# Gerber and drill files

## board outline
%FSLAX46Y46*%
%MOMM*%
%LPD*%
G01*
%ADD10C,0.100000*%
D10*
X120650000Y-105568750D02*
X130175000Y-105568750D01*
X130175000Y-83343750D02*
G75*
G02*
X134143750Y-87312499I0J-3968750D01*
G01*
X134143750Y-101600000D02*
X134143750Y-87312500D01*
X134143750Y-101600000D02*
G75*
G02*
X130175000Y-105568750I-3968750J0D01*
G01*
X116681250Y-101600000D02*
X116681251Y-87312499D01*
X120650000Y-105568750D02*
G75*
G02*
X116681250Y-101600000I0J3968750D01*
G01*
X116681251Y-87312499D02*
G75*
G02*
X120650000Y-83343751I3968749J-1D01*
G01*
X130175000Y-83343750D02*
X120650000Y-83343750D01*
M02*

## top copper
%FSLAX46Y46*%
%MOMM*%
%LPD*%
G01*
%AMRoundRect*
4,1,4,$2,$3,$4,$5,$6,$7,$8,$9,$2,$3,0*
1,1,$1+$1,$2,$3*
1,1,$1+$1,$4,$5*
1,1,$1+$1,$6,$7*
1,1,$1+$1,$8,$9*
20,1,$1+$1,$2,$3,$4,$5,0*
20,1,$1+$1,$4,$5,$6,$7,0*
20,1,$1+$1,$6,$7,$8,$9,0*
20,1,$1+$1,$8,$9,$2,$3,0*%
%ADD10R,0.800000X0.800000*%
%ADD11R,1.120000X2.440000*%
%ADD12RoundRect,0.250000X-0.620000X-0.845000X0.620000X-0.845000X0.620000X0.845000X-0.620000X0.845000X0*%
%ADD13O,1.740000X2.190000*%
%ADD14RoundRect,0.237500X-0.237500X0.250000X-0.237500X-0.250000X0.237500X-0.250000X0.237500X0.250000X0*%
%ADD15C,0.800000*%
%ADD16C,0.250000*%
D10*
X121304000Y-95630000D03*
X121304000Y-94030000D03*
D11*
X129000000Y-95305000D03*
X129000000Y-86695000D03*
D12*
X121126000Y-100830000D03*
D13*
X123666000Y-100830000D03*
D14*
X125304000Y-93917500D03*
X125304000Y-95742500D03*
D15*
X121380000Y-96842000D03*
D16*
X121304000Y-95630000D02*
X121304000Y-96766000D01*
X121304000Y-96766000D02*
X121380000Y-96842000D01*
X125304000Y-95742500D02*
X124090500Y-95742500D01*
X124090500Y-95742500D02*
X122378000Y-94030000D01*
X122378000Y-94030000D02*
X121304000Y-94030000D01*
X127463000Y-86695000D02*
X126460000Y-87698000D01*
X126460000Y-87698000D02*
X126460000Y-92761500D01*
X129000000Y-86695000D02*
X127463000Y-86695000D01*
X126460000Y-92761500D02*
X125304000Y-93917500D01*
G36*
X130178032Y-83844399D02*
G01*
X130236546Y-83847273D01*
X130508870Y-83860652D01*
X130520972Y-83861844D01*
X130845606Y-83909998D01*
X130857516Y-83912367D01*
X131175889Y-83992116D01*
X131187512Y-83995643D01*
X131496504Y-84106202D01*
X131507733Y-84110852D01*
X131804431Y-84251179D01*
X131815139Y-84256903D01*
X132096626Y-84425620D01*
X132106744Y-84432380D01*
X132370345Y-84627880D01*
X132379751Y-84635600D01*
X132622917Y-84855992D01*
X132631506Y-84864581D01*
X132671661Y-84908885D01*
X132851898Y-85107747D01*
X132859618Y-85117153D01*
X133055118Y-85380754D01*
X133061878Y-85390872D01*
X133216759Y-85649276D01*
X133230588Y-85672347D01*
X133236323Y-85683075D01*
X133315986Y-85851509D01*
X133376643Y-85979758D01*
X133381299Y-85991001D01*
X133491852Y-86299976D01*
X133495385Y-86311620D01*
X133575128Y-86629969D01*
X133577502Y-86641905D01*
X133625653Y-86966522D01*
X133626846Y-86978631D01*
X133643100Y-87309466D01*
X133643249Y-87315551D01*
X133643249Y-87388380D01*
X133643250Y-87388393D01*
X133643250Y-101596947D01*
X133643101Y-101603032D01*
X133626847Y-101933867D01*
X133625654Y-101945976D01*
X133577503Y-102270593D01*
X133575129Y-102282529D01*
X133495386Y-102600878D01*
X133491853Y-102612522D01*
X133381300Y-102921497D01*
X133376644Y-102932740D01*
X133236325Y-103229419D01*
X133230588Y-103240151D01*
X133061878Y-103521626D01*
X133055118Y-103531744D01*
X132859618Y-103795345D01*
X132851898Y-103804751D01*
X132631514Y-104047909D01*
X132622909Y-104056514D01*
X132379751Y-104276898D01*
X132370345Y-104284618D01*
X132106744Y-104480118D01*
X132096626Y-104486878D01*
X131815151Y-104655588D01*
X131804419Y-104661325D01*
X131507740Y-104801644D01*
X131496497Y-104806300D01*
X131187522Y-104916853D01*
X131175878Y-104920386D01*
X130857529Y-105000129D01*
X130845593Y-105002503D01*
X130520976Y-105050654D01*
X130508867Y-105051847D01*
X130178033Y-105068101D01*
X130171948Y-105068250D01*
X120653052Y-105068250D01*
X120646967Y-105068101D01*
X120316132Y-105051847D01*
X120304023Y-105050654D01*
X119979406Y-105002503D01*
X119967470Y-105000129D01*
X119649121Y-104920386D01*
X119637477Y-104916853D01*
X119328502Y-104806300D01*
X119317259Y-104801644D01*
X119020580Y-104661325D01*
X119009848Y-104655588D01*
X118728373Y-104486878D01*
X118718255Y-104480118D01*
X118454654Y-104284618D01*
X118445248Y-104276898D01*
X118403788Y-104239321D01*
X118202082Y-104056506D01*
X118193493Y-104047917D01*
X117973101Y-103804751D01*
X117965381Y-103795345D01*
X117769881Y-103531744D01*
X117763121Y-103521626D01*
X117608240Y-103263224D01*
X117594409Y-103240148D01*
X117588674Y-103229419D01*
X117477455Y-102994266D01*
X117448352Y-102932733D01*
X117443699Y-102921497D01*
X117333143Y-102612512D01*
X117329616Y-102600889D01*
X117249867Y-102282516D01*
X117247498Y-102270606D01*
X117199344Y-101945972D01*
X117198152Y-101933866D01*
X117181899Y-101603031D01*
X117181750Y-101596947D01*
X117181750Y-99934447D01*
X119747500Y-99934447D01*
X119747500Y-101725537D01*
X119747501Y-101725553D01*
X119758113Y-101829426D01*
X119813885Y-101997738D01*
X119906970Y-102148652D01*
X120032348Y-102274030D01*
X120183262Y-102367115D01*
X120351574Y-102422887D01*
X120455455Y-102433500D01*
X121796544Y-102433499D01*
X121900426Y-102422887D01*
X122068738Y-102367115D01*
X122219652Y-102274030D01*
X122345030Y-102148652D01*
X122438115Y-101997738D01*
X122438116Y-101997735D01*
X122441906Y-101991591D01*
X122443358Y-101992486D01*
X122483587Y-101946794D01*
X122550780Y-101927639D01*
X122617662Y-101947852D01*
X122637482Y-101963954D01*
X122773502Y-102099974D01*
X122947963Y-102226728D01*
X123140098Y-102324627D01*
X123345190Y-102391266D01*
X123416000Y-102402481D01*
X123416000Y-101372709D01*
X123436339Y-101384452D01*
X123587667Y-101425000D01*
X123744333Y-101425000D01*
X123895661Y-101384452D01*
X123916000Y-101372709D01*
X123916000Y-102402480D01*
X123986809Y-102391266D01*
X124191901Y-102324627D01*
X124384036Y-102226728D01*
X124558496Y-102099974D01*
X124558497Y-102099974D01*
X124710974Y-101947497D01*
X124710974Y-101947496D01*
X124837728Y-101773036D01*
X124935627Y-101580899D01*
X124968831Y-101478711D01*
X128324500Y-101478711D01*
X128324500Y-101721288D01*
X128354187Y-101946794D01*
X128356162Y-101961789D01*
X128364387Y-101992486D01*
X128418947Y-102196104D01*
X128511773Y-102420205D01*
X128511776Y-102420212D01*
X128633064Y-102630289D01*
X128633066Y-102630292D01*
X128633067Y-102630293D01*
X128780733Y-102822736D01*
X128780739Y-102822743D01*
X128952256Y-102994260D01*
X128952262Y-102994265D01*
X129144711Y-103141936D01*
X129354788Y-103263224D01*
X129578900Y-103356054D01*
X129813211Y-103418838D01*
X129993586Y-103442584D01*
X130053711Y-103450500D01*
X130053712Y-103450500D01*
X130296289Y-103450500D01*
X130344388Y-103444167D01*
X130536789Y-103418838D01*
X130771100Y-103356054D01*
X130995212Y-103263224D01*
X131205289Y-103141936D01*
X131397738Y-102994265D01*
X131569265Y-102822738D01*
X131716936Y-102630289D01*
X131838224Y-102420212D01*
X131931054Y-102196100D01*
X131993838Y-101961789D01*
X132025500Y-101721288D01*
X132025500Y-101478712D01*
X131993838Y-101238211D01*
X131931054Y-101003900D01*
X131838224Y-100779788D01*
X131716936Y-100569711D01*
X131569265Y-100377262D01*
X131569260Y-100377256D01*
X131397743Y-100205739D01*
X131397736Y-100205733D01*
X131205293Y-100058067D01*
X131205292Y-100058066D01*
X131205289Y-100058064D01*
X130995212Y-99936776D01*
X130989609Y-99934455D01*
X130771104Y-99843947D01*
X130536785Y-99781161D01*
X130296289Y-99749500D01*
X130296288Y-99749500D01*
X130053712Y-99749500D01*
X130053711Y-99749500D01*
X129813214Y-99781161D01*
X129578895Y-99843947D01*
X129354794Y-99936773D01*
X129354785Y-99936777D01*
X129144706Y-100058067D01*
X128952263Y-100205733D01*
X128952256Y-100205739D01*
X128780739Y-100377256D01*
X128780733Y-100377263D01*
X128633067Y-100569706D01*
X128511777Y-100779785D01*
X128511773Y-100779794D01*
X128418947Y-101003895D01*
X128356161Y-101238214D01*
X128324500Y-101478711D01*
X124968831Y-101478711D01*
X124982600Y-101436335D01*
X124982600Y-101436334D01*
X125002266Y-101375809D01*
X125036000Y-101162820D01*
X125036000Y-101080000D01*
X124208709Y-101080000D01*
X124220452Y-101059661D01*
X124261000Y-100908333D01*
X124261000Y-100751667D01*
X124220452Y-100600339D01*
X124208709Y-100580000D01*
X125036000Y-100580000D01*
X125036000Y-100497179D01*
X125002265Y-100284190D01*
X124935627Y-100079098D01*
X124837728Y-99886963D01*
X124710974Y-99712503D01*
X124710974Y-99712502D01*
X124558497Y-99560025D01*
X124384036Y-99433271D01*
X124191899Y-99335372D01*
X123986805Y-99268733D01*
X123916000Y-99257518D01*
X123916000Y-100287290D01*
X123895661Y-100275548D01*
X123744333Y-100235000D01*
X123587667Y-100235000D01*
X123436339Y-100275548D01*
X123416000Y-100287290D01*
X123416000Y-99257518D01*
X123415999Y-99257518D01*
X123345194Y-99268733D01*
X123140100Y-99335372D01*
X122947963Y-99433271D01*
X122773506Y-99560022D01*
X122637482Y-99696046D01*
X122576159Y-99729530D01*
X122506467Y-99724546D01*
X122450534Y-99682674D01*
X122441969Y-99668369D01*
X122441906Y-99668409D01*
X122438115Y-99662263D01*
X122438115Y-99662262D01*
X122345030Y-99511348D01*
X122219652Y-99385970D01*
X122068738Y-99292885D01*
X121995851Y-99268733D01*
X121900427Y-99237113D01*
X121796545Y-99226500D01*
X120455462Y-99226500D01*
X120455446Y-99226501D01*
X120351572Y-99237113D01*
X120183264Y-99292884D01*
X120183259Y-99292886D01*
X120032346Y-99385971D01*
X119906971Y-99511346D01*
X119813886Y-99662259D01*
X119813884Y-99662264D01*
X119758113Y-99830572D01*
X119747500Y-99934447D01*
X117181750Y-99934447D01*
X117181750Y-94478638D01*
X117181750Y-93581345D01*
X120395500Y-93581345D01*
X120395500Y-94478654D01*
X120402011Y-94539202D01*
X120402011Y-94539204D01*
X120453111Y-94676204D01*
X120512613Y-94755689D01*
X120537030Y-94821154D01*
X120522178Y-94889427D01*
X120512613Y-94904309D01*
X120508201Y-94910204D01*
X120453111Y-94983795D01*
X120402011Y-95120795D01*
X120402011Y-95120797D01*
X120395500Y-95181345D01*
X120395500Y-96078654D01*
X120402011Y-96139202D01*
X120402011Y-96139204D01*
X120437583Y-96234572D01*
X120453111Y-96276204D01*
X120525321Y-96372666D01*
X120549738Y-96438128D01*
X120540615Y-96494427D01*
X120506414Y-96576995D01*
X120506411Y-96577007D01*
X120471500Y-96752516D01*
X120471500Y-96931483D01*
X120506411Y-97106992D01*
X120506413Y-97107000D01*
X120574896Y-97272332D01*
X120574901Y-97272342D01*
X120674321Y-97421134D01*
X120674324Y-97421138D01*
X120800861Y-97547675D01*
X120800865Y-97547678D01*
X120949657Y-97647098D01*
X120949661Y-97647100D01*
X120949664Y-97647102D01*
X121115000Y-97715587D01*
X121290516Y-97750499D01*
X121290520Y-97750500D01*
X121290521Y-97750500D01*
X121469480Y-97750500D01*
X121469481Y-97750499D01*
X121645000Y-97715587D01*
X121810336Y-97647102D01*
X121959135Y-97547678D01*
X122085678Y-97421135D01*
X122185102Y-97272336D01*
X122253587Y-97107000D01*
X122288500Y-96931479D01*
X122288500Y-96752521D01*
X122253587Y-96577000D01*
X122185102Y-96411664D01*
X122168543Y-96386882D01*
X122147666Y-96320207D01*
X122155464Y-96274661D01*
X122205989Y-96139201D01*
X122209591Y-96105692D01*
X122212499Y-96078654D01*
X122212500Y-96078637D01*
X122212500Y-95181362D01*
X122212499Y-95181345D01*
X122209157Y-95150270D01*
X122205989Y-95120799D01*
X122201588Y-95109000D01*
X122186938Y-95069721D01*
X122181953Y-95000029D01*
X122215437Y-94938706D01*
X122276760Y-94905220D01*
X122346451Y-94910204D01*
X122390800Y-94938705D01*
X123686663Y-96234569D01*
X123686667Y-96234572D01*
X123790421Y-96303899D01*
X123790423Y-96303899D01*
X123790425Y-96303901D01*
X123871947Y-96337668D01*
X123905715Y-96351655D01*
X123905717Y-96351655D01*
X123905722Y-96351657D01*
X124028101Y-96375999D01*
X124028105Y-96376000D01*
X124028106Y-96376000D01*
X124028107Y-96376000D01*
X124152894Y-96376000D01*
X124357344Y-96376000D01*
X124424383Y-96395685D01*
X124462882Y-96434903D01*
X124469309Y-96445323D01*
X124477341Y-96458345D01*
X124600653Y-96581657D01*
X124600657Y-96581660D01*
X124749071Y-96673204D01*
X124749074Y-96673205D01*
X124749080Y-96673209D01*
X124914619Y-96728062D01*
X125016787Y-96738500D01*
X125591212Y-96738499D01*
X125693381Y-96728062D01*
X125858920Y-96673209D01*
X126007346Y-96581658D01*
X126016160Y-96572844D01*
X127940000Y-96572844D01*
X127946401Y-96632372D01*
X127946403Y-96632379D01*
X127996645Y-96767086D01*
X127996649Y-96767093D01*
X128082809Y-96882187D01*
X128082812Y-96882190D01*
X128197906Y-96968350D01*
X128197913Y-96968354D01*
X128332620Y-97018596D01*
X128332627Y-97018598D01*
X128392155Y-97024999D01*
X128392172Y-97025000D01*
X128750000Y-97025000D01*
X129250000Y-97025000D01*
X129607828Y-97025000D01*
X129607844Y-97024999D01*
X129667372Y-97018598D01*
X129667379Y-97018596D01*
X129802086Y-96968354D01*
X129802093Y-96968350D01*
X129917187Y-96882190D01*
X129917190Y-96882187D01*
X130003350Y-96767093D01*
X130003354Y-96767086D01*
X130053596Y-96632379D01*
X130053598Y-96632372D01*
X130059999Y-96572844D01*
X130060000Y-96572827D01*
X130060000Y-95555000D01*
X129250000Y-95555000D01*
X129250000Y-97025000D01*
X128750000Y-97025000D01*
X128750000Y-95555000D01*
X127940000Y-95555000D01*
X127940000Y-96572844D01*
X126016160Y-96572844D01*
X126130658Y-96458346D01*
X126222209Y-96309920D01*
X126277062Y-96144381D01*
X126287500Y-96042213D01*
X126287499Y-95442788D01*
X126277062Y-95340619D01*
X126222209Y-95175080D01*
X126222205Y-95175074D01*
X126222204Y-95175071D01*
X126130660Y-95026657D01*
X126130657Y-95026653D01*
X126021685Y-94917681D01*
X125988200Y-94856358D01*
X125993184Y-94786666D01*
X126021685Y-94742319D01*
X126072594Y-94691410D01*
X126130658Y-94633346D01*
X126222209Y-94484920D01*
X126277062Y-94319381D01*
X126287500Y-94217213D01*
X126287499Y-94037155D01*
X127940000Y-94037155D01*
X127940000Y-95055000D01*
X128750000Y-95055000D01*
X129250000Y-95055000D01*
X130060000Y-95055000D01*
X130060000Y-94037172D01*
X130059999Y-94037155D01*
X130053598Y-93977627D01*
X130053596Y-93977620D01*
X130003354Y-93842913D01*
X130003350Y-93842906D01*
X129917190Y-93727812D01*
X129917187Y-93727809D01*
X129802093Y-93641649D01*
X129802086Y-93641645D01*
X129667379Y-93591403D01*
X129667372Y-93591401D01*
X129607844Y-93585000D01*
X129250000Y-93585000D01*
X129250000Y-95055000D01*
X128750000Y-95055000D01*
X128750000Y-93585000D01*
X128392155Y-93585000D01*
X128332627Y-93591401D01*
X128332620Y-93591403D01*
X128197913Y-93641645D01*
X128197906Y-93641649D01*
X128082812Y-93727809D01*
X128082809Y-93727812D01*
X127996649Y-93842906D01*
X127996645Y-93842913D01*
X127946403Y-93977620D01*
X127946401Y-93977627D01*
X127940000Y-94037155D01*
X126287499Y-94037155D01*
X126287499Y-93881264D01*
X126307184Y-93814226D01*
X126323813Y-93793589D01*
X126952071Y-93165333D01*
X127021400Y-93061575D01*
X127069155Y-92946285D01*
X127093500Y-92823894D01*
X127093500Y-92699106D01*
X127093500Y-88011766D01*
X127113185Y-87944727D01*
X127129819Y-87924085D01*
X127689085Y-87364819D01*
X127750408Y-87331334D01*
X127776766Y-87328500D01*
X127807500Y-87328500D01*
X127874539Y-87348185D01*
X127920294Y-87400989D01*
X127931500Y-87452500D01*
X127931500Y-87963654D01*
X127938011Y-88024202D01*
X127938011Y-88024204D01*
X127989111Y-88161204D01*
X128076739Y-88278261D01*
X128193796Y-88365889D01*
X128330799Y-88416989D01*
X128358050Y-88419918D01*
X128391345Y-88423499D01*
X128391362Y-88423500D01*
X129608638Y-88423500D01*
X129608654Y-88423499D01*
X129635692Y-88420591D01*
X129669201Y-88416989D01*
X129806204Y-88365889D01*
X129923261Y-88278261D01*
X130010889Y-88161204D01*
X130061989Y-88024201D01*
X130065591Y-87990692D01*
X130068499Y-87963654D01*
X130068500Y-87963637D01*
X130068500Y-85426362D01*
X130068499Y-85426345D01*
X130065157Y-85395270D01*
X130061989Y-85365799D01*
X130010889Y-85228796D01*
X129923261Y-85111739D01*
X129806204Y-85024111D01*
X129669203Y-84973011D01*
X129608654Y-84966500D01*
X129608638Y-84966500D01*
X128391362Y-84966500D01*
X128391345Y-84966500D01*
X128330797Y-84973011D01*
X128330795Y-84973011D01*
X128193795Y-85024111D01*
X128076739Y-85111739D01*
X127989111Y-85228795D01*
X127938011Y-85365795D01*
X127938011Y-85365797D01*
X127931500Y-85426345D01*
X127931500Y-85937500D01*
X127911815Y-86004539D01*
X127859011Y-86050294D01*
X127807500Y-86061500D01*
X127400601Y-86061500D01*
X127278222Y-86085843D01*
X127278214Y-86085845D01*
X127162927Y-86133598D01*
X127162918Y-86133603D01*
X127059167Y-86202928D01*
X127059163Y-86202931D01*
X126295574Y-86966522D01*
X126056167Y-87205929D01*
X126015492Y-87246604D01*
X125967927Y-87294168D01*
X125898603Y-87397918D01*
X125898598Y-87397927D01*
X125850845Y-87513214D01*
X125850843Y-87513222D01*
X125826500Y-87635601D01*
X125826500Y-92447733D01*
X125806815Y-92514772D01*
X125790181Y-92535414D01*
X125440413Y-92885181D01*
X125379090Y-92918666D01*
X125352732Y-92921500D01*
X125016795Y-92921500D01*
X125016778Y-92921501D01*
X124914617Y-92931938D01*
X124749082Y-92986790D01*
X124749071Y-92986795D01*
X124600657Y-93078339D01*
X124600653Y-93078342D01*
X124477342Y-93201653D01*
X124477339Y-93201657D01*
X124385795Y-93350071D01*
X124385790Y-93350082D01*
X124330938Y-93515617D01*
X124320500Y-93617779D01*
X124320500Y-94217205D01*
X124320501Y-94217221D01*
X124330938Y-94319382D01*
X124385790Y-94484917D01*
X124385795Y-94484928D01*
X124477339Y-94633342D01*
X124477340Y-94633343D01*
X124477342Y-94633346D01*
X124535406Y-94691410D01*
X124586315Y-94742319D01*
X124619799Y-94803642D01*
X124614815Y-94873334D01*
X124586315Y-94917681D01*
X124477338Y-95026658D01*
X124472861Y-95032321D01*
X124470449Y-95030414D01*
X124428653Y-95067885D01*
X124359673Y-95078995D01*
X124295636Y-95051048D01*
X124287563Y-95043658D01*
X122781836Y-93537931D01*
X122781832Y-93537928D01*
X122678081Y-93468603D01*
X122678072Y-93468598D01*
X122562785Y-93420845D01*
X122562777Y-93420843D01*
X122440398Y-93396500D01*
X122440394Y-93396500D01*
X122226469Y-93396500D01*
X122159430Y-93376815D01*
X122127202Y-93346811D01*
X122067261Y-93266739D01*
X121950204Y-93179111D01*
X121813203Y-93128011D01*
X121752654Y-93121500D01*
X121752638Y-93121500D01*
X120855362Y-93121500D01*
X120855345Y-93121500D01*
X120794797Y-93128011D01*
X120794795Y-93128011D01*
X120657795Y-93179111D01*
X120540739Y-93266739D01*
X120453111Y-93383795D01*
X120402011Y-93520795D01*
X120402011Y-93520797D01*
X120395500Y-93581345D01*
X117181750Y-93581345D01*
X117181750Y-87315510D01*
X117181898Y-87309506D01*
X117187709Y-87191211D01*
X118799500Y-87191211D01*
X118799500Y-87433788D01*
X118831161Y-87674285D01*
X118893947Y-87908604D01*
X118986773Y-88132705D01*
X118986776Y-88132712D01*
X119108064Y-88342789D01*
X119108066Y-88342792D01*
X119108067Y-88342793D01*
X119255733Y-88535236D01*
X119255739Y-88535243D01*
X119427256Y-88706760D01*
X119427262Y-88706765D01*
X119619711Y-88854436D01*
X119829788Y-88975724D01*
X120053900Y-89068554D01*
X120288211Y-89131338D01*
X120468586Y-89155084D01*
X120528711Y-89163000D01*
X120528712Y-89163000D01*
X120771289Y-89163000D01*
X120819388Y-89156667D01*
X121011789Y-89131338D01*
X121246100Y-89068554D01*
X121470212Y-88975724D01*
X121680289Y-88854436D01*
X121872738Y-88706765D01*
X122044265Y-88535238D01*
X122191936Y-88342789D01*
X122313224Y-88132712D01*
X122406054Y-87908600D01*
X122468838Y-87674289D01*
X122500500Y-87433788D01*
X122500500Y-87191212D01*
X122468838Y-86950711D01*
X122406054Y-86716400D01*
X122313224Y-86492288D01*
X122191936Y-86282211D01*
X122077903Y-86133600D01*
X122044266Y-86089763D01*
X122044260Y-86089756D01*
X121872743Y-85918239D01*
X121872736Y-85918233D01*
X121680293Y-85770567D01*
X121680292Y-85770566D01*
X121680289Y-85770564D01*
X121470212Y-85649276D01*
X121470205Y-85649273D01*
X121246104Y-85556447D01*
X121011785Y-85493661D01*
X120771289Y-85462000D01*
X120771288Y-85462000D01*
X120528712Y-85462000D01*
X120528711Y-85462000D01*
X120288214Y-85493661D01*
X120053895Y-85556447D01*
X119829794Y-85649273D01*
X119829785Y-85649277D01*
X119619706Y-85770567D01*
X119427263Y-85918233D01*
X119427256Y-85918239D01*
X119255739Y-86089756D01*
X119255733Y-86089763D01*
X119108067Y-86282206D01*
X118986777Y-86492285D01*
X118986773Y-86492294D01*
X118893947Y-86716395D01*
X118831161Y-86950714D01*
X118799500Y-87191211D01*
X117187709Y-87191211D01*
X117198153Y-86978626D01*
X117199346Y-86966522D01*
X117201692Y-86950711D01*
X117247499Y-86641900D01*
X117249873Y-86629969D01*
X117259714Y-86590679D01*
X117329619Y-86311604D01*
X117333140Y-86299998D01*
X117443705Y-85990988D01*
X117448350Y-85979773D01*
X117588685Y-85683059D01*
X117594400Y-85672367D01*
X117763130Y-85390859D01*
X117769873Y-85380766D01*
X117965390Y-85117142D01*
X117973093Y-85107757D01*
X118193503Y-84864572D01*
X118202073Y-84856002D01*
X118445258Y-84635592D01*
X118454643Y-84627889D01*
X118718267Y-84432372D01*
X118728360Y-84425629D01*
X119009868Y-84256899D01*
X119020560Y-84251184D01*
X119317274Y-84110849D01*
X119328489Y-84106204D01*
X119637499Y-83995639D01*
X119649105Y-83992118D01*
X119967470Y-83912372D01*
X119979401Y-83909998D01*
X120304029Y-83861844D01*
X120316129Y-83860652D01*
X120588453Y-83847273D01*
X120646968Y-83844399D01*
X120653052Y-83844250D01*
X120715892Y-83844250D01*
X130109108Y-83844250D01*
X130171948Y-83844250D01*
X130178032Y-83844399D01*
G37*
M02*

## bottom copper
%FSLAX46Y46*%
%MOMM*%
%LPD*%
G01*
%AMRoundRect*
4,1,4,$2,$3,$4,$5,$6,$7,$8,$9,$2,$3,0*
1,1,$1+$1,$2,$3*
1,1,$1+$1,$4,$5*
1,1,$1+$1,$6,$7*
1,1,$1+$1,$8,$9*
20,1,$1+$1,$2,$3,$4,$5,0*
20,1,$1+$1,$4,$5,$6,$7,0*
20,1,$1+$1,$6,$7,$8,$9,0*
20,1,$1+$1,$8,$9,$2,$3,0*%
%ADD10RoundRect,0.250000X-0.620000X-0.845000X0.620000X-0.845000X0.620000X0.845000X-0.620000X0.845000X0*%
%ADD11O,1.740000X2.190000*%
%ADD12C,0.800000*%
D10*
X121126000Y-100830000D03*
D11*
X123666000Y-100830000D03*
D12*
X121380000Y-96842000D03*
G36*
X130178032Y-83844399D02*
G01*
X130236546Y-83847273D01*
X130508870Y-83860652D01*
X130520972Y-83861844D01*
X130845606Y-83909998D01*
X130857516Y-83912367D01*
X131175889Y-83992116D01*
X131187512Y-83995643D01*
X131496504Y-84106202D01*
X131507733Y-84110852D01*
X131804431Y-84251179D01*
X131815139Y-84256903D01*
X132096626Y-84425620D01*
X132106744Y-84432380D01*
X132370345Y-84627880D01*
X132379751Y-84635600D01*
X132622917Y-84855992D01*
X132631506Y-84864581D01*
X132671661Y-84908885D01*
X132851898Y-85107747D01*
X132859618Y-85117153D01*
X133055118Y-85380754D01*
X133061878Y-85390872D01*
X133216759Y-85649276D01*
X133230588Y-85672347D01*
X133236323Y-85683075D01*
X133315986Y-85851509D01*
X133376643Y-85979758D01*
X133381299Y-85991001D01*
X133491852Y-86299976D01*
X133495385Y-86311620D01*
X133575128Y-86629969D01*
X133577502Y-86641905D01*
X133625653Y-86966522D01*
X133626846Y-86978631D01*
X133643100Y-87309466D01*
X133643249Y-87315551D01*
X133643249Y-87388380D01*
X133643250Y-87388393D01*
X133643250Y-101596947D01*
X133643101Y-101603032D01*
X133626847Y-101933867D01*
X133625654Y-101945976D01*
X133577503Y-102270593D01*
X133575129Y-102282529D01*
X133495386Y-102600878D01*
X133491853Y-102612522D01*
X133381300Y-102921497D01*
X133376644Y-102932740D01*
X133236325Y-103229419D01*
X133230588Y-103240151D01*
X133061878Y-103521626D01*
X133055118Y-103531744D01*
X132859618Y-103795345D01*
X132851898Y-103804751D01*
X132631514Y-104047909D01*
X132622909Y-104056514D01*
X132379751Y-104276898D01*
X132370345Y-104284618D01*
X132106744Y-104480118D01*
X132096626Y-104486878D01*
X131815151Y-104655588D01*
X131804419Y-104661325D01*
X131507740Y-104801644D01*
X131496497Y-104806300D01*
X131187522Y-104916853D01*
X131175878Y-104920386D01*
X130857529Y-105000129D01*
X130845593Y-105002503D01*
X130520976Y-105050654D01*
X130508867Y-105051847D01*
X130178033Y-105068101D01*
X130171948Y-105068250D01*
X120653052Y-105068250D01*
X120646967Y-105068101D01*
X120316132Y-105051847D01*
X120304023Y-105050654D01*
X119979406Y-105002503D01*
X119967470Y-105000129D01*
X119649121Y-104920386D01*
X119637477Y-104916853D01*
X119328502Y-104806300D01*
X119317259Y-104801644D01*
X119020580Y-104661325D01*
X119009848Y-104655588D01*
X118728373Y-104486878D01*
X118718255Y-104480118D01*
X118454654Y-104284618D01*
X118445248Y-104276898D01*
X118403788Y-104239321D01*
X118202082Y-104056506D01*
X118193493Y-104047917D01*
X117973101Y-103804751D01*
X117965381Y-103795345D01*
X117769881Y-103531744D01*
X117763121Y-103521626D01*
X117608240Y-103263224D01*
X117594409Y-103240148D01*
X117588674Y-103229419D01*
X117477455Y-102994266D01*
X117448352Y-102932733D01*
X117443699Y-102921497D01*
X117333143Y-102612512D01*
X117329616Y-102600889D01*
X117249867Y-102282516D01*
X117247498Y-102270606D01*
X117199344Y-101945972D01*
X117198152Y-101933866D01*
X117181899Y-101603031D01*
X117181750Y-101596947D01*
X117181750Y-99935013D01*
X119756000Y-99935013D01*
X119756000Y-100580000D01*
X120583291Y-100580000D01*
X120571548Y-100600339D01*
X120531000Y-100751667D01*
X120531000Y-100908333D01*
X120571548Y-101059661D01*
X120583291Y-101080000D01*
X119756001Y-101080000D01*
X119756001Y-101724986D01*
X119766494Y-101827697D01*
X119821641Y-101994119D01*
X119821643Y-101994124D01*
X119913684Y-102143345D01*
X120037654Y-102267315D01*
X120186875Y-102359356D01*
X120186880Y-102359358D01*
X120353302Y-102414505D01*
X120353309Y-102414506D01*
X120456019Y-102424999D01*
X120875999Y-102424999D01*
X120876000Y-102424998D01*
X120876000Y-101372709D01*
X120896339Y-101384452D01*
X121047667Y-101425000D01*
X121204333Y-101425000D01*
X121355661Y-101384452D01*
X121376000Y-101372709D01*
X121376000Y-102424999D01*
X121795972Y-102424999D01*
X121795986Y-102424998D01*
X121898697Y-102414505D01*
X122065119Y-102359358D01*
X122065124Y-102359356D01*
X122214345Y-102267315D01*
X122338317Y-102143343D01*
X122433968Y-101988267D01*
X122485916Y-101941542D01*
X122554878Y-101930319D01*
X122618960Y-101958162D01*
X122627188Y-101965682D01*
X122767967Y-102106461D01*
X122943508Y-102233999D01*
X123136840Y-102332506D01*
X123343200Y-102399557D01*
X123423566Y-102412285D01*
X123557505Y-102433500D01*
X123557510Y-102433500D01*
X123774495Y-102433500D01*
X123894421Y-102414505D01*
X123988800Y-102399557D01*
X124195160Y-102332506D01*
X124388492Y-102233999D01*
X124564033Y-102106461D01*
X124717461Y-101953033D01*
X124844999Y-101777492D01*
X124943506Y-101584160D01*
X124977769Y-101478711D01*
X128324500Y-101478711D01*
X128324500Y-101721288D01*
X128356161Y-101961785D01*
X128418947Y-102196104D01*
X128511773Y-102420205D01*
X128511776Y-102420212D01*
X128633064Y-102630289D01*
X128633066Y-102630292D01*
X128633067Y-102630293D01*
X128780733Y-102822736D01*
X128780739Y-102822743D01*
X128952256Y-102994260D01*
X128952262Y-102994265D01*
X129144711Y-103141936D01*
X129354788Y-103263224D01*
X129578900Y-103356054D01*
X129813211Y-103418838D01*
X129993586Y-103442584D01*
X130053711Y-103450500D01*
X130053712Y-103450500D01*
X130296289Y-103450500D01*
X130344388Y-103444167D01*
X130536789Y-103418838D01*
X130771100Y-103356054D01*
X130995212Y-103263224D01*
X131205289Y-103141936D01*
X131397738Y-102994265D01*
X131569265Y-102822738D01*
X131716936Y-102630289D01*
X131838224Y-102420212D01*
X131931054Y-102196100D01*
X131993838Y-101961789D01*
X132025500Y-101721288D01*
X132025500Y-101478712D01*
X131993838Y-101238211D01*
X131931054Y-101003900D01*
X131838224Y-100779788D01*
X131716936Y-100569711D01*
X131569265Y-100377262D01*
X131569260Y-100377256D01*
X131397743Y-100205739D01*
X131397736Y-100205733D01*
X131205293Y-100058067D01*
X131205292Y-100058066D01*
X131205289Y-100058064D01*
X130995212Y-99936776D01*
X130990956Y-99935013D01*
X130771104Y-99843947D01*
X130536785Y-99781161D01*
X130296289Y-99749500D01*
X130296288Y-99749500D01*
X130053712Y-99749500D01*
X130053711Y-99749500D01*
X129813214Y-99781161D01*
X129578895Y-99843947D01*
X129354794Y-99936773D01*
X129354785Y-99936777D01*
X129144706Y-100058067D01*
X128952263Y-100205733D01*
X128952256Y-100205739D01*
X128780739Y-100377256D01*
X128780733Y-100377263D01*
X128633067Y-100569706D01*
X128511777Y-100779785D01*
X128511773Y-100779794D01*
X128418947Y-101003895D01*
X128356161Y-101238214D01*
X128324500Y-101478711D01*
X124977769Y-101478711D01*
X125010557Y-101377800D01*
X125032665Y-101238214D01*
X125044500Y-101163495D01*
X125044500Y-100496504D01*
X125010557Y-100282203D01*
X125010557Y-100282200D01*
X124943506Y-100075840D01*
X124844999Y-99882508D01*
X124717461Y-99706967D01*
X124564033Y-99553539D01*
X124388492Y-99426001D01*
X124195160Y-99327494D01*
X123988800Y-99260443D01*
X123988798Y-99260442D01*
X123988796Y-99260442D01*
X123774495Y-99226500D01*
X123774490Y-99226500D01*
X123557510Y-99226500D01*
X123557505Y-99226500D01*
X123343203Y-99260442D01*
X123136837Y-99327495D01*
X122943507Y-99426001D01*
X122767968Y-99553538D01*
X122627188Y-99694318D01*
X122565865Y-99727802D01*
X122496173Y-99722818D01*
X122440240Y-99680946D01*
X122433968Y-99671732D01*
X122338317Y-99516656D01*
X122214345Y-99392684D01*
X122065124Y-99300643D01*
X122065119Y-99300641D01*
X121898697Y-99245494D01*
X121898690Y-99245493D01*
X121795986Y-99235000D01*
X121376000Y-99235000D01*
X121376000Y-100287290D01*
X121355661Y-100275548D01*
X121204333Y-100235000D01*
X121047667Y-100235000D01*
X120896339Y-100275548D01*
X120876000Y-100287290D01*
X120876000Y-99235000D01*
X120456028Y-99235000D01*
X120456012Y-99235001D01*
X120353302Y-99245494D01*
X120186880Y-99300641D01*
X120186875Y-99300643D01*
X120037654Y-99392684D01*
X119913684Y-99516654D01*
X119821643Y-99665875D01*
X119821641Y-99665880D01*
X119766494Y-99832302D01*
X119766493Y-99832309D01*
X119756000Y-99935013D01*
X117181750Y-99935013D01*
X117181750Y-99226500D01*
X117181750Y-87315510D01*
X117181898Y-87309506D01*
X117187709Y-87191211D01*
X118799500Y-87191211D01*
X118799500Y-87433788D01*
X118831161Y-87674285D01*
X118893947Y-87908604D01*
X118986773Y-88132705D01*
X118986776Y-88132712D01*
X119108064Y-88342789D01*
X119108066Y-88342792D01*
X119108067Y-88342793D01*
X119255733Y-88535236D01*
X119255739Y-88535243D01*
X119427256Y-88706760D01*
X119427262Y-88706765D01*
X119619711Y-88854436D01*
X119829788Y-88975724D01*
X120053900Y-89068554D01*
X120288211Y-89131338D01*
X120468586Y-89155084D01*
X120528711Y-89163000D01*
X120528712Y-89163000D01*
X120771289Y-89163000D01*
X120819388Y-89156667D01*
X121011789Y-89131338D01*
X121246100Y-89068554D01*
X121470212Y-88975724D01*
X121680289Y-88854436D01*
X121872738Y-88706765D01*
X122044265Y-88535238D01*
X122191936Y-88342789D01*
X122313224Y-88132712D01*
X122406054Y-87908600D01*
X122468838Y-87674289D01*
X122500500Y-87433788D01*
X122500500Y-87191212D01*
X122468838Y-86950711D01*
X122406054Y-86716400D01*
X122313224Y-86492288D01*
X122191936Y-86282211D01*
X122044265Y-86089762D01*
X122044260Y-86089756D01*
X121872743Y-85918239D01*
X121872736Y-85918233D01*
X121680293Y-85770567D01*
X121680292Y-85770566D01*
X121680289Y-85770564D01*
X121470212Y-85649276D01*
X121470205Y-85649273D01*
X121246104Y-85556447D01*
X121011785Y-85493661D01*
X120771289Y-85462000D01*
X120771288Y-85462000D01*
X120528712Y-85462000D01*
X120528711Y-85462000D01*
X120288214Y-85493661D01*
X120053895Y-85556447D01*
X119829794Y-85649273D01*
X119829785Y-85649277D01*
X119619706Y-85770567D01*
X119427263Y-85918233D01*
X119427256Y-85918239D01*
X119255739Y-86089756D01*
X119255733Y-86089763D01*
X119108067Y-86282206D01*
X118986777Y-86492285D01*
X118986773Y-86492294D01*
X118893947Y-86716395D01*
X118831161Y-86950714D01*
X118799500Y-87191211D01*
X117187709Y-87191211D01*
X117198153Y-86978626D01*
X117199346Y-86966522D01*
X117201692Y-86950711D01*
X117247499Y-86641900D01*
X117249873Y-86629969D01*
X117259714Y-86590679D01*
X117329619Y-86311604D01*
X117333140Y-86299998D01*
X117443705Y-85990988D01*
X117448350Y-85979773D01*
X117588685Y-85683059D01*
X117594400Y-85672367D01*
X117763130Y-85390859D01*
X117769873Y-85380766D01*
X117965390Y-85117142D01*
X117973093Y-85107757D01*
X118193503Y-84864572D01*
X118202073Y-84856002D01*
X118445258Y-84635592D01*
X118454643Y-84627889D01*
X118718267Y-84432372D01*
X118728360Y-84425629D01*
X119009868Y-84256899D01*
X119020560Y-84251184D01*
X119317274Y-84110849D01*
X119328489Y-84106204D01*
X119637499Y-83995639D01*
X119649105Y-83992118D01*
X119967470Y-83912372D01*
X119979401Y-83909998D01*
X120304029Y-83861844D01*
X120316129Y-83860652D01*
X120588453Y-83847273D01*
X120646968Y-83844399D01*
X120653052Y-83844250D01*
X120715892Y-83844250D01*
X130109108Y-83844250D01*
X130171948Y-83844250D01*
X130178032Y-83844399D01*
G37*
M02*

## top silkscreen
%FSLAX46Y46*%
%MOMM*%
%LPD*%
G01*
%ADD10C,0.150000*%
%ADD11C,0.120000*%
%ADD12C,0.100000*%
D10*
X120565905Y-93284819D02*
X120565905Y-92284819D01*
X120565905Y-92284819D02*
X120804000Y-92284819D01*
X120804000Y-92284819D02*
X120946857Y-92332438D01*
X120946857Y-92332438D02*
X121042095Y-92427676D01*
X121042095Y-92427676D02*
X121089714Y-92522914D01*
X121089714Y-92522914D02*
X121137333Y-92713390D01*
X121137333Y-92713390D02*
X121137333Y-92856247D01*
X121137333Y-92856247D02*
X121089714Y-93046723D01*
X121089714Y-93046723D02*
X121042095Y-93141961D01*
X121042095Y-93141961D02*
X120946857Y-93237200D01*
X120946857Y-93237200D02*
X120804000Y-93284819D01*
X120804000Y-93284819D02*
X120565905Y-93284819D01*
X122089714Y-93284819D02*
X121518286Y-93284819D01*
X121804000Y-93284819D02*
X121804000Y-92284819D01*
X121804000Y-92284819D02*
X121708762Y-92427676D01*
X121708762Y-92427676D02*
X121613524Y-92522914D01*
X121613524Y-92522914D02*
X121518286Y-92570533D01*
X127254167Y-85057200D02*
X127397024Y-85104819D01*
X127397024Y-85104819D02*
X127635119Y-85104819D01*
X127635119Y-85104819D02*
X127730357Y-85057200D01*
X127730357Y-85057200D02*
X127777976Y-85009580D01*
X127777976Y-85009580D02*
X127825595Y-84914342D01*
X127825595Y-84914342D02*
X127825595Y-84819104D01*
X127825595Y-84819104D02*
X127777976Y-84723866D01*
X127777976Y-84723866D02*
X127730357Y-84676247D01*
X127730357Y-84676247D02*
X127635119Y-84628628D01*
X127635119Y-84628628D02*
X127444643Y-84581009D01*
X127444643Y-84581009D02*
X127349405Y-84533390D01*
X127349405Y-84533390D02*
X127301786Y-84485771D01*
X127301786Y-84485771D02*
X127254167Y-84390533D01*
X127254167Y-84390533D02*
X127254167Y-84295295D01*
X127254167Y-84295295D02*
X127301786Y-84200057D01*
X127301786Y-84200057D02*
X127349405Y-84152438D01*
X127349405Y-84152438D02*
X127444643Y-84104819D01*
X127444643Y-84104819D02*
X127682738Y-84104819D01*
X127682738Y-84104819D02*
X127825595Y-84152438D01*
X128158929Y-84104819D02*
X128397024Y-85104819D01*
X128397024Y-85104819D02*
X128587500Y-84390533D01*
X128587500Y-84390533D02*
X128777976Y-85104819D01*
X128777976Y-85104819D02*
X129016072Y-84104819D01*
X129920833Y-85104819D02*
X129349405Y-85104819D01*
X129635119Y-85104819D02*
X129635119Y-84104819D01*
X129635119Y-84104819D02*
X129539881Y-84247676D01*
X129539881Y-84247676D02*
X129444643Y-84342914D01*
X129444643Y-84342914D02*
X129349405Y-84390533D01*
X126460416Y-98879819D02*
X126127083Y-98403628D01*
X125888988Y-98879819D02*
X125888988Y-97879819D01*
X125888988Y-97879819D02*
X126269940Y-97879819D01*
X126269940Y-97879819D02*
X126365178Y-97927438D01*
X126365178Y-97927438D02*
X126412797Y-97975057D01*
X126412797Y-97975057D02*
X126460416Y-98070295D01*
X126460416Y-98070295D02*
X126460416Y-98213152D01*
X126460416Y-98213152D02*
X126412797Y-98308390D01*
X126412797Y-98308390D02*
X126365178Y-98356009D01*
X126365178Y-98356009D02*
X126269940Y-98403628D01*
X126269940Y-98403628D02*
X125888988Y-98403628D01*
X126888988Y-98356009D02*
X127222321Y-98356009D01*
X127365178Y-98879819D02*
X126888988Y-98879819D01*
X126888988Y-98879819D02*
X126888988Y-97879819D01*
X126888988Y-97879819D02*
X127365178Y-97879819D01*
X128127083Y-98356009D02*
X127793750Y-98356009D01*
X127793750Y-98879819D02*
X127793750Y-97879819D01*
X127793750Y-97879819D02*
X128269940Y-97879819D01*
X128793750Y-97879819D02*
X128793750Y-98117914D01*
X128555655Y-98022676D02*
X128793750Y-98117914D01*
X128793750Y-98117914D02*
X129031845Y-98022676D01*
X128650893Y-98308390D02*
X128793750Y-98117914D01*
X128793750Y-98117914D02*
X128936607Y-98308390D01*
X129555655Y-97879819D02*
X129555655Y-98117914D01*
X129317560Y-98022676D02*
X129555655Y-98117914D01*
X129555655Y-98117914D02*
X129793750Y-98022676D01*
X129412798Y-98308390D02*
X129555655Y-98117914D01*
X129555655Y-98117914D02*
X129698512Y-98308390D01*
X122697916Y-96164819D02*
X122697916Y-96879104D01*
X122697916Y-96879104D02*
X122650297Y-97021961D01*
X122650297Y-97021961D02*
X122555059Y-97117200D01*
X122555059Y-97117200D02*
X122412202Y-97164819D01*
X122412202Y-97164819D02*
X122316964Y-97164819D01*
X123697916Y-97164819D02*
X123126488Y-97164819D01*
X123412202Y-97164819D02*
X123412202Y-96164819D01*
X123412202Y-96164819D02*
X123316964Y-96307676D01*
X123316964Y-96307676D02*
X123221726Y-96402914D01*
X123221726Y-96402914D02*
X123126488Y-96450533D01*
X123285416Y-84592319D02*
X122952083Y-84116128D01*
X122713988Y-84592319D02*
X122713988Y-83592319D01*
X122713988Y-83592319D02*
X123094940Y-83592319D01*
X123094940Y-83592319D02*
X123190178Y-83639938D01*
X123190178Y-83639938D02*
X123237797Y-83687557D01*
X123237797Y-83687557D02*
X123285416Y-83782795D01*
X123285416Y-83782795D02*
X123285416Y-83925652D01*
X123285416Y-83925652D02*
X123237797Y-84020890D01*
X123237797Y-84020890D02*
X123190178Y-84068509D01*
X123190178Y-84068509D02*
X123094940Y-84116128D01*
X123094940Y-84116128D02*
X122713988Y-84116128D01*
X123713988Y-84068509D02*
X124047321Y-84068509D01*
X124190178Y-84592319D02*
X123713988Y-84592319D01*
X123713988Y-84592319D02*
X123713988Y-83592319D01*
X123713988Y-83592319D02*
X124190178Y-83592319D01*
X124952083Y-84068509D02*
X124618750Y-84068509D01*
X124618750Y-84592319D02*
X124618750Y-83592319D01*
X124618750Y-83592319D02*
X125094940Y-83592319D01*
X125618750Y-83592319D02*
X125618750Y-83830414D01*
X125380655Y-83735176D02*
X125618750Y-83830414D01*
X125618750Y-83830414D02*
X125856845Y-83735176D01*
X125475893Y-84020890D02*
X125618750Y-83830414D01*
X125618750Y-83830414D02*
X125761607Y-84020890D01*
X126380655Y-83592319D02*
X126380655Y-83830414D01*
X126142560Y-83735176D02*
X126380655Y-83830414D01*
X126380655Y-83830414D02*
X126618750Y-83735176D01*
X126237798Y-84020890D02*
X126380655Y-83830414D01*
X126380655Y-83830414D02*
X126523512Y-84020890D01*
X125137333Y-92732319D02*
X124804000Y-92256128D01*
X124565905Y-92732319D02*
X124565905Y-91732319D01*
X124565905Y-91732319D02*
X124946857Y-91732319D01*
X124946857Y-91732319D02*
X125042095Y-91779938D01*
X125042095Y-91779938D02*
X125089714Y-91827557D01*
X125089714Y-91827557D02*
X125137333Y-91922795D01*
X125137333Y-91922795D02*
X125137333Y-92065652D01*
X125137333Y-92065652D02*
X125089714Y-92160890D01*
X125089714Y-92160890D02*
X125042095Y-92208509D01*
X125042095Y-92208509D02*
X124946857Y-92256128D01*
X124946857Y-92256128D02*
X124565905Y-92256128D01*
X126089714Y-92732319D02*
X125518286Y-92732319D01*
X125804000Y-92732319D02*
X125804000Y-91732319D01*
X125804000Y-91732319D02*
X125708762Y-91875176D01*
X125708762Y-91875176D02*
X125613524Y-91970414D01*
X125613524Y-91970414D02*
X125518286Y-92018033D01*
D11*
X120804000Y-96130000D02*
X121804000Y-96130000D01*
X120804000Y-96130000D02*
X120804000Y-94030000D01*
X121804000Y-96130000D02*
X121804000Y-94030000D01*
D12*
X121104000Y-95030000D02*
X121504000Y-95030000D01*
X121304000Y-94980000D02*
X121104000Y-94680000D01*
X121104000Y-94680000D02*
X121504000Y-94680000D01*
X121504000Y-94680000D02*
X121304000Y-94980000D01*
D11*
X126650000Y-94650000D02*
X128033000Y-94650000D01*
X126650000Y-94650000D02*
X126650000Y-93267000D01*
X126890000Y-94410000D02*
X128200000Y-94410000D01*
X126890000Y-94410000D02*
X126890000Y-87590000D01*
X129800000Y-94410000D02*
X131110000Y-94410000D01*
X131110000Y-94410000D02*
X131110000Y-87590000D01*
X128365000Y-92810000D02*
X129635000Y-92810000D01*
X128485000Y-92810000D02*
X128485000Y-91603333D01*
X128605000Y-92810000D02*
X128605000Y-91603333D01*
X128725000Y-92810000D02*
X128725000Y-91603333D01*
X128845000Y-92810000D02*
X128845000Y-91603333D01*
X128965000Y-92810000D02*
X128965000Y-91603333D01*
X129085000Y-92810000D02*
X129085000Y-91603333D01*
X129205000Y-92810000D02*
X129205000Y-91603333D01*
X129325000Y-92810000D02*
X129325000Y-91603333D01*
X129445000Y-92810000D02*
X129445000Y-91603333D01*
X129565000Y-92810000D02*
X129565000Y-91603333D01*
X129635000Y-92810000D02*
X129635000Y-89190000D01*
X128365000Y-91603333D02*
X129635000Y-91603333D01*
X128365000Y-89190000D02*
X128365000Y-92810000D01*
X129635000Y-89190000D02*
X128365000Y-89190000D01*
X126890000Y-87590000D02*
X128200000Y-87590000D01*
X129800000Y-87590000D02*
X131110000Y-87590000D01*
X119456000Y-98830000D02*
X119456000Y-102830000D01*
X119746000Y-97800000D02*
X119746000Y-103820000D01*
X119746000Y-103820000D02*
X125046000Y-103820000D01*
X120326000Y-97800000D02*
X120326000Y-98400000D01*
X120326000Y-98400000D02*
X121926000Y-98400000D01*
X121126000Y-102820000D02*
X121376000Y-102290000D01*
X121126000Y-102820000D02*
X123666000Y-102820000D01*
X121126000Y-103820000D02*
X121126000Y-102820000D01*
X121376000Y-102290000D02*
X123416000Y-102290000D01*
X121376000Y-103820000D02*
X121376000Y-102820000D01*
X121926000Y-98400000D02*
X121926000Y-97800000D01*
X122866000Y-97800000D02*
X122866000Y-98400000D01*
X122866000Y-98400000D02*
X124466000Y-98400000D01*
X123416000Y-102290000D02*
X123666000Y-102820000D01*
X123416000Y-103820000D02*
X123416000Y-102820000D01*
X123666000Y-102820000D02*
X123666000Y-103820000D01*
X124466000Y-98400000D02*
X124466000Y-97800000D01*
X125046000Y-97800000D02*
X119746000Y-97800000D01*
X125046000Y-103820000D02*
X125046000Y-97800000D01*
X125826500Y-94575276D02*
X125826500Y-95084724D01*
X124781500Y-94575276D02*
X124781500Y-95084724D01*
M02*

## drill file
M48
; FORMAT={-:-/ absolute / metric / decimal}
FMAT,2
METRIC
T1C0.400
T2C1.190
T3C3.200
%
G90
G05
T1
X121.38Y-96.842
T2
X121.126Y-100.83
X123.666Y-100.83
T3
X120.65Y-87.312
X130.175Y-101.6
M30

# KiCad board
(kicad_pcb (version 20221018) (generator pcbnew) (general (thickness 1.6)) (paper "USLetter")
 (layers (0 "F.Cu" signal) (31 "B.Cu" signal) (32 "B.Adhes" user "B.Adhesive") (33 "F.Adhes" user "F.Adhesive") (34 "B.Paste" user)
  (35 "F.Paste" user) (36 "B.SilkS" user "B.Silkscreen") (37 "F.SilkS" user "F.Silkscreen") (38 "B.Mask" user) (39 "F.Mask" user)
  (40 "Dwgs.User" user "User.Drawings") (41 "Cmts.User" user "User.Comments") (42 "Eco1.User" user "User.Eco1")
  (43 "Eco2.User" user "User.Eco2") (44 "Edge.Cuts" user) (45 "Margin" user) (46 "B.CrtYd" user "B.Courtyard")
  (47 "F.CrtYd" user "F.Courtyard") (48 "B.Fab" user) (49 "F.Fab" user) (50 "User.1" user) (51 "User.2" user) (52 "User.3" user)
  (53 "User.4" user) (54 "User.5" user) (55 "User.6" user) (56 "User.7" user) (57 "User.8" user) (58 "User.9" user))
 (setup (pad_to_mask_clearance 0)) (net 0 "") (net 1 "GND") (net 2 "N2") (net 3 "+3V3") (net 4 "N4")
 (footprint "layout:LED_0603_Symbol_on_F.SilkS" (layer "F.Cu") (at 121.304 94.83 90)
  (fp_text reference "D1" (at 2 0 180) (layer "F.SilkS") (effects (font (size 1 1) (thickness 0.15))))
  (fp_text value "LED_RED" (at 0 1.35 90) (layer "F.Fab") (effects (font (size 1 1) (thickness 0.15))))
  (fp_line (start -1.3 -0.5) (end -1.3 0.5) (stroke (width 0.12) (type solid)) (layer "F.SilkS"))
  (fp_line (start -1.3 -0.5) (end 0.8 -0.5) (stroke (width 0.12) (type solid)) (layer "F.SilkS"))
  (fp_line (start -1.3 0.5) (end 0.8 0.5) (stroke (width 0.12) (type solid)) (layer "F.SilkS"))
  (fp_line (start -0.2 -0.2) (end -0.2 0.2) (stroke (width 0.1) (type solid)) (layer "F.SilkS"))
  (fp_line (start -0.15 0) (end 0.15 -0.2) (stroke (width 0.1) (type solid)) (layer "F.SilkS"))
  (fp_line (start 0.15 -0.2) (end 0.15 0.2) (stroke (width 0.1) (type solid)) (layer "F.SilkS"))
  (fp_line (start 0.15 0.2) (end -0.15 0) (stroke (width 0.1) (type solid)) (layer "F.SilkS"))
  (pad "1" smd rect (at -0.8 0 270) (size 0.8 0.8) (layers "F.Cu" "F.Paste" "F.Mask") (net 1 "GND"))
  (pad "2" smd rect (at 0.8 0 270) (size 0.8 0.8) (layers "F.Cu" "F.Paste" "F.Mask") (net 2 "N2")))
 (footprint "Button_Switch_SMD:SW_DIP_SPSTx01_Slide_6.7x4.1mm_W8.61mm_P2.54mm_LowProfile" (layer "F.Cu") (at 129 91 90)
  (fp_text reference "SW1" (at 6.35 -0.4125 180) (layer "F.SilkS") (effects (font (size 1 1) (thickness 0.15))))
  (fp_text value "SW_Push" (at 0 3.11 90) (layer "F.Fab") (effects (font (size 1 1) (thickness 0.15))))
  (fp_line (start -3.65 -2.35) (end -3.65 -0.967) (stroke (width 0.12) (type solid)) (layer "F.SilkS"))
  (fp_line (start -3.65 -2.35) (end -2.267 -2.35) (stroke (width 0.12) (type solid)) (layer "F.SilkS"))
  (fp_line (start -3.41 -2.11) (end -3.41 -0.8) (stroke (width 0.12) (type solid)) (layer "F.SilkS"))
  (fp_line (start -3.41 -2.11) (end 3.41 -2.11) (stroke (width 0.12) (type solid)) (layer "F.SilkS"))
  (fp_line (start -3.41 0.8) (end -3.41 2.11) (stroke (width 0.12) (type solid)) (layer "F.SilkS"))
  (fp_line (start -3.41 2.11) (end 3.41 2.11) (stroke (width 0.12) (type solid)) (layer "F.SilkS"))
  (fp_line (start -1.81 -0.635) (end -1.81 0.635) (stroke (width 0.12) (type solid)) (layer "F.SilkS"))
  (fp_line (start -1.81 -0.515) (end -0.603333 -0.515) (stroke (width 0.12) (type solid)) (layer "F.SilkS"))
  (fp_line (start -1.81 -0.395) (end -0.603333 -0.395) (stroke (width 0.12) (type solid)) (layer "F.SilkS"))
  (fp_line (start -1.81 -0.275) (end -0.603333 -0.275) (stroke (width 0.12) (type solid)) (layer "F.SilkS"))
  (fp_line (start -1.81 -0.155) (end -0.603333 -0.155) (stroke (width 0.12) (type solid)) (layer "F.SilkS"))
  (fp_line (start -1.81 -0.035) (end -0.603333 -0.035) (stroke (width 0.12) (type solid)) (layer "F.SilkS"))
  (fp_line (start -1.81 0.085) (end -0.603333 0.085) (stroke (width 0.12) (type solid)) (layer "F.SilkS"))
  (fp_line (start -1.81 0.205) (end -0.603333 0.205) (stroke (width 0.12) (type solid)) (layer "F.SilkS"))
  (fp_line (start -1.81 0.325) (end -0.603333 0.325) (stroke (width 0.12) (type solid)) (layer "F.SilkS"))
  (fp_line (start -1.81 0.445) (end -0.603333 0.445) (stroke (width 0.12) (type solid)) (layer "F.SilkS"))
  (fp_line (start -1.81 0.565) (end -0.603333 0.565) (stroke (width 0.12) (type solid)) (layer "F.SilkS"))
  (fp_line (start -1.81 0.635) (end 1.81 0.635) (stroke (width 0.12) (type solid)) (layer "F.SilkS"))
  (fp_line (start -0.603333 -0.635) (end -0.603333 0.635) (stroke (width 0.12) (type solid)) (layer "F.SilkS"))
  (fp_line (start 1.81 -0.635) (end -1.81 -0.635) (stroke (width 0.12) (type solid)) (layer "F.SilkS"))
  (fp_line (start 1.81 0.635) (end 1.81 -0.635) (stroke (width 0.12) (type solid)) (layer "F.SilkS"))
  (fp_line (start 3.41 -2.11) (end 3.41 -0.8) (stroke (width 0.12) (type solid)) (layer "F.SilkS"))
  (fp_line (start 3.41 0.8) (end 3.41 2.11) (stroke (width 0.12) (type solid)) (layer "F.SilkS"))
  (pad "1" smd rect (at -4.305 0 90) (size 2.44 1.12) (layers "F.Cu" "F.Paste" "F.Mask") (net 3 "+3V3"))
  (pad "2" smd rect (at 4.305 0 90) (size 2.44 1.12) (layers "F.Cu" "F.Paste" "F.Mask") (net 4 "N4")))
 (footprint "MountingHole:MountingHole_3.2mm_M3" (layer "F.Cu") (at 130.175 101.6)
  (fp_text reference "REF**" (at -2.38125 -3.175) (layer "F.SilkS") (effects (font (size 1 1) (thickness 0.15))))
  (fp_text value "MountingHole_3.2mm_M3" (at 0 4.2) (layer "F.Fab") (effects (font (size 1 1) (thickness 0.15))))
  (pad "" np_thru_hole circle (at 0 0) (size 3.2 3.2) (drill 3.2) (layers "*.Cu" "*.Mask")))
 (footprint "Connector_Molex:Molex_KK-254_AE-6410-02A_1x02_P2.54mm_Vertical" (layer "F.Cu") (at 121.126 100.83)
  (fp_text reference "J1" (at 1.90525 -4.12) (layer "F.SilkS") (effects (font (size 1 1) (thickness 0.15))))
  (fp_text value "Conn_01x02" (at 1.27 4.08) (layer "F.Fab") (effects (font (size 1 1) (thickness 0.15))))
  (fp_line (start -1.67 -2) (end -1.67 2) (stroke (width 0.12) (type solid)) (layer "F.SilkS"))
  (fp_line (start -1.38 -3.03) (end -1.38 2.99) (stroke (width 0.12) (type solid)) (layer "F.SilkS"))
  (fp_line (start -1.38 2.99) (end 3.92 2.99) (stroke (width 0.12) (type solid)) (layer "F.SilkS"))
  (fp_line (start -0.8 -3.03) (end -0.8 -2.43) (stroke (width 0.12) (type solid)) (layer "F.SilkS"))
  (fp_line (start -0.8 -2.43) (end 0.8 -2.43) (stroke (width 0.12) (type solid)) (layer "F.SilkS"))
  (fp_line (start 0 1.99) (end 0.25 1.46) (stroke (width 0.12) (type solid)) (layer "F.SilkS"))
  (fp_line (start 0 1.99) (end 2.54 1.99) (stroke (width 0.12) (type solid)) (layer "F.SilkS"))
  (fp_line (start 0 2.99) (end 0 1.99) (stroke (width 0.12) (type solid)) (layer "F.SilkS"))
  (fp_line (start 0.25 1.46) (end 2.29 1.46) (stroke (width 0.12) (type solid)) (layer "F.SilkS"))
  (fp_line (start 0.25 2.99) (end 0.25 1.99) (stroke (width 0.12) (type solid)) (layer "F.SilkS"))
  (fp_line (start 0.8 -2.43) (end 0.8 -3.03) (stroke (width 0.12) (type solid)) (layer "F.SilkS"))
  (fp_line (start 1.74 -3.03) (end 1.74 -2.43) (stroke (width 0.12) (type solid)) (layer "F.SilkS"))
  (fp_line (start 1.74 -2.43) (end 3.34 -2.43) (stroke (width 0.12) (type solid)) (layer "F.SilkS"))
  (fp_line (start 2.29 1.46) (end 2.54 1.99) (stroke (width 0.12) (type solid)) (layer "F.SilkS"))
  (fp_line (start 2.29 2.99) (end 2.29 1.99) (stroke (width 0.12) (type solid)) (layer "F.SilkS"))
  (fp_line (start 2.54 1.99) (end 2.54 2.99) (stroke (width 0.12) (type solid)) (layer "F.SilkS"))
  (fp_line (start 3.34 -2.43) (end 3.34 -3.03) (stroke (width 0.12) (type solid)) (layer "F.SilkS"))
  (fp_line (start 3.92 -3.03) (end -1.38 -3.03) (stroke (width 0.12) (type solid)) (layer "F.SilkS"))
  (fp_line (start 3.92 2.99) (end 3.92 -3.03) (stroke (width 0.12) (type solid)) (layer "F.SilkS"))
  (pad "1" thru_hole roundrect (at 0 0) (size 1.74 2.19) (drill 1.19) (layers "*.Cu" "*.Mask") (roundrect_rratio 0.143678) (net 1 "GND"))
  (pad "2" thru_hole oval (at 2.54 0) (size 1.74 2.19) (drill 1.19) (layers "*.Cu" "*.Mask") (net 3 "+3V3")))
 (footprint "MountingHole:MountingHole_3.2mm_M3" (layer "F.Cu") (at 120.65 87.3125)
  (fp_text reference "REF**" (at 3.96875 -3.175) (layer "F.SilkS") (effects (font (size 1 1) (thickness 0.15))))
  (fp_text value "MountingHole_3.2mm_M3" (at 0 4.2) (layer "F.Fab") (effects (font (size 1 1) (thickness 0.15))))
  (pad "" np_thru_hole circle (at 0 0) (size 3.2 3.2) (drill 3.2) (layers "*.Cu" "*.Mask")))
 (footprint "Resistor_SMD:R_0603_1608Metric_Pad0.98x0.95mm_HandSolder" (layer "F.Cu") (at 125.304 94.83 -90)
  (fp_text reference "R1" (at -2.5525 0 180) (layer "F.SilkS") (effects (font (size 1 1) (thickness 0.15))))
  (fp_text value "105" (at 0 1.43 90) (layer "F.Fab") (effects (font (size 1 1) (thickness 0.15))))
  (fp_line (start -0.254724 -0.5225) (end 0.254724 -0.5225) (stroke (width 0.12) (type solid)) (layer "F.SilkS"))
  (fp_line (start -0.254724 0.5225) (end 0.254724 0.5225) (stroke (width 0.12) (type solid)) (layer "F.SilkS"))
  (pad "1" smd roundrect (at -0.9125 0 270) (size 0.975 0.95) (layers "F.Cu" "F.Paste" "F.Mask") (roundrect_rratio 0.25) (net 4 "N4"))
  (pad "2" smd roundrect (at 0.9125 0 270) (size 0.975 0.95) (layers "F.Cu" "F.Paste" "F.Mask") (roundrect_rratio 0.25) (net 2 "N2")))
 (gr_line (start 120.65 105.56875) (end 130.175 105.56875) (stroke (width 0.1) (type default)) (layer "Edge.Cuts"))
 (gr_arc (start 130.175 83.34375) (mid 132.98133 84.50617) (end 134.143749 87.312499) (stroke (width 0.1) (type default))
  (layer "Edge.Cuts"))
 (gr_line (start 134.14375 101.6) (end 134.14375 87.3125) (stroke (width 0.1) (type default)) (layer "Edge.Cuts"))
 (gr_arc (start 134.14375 101.6) (mid 132.98133 104.40633) (end 130.175 105.56875) (stroke (width 0.1) (type default)) (layer "Edge.Cuts"))
 (gr_line (start 116.68125 101.6) (end 116.681251 87.312499) (stroke (width 0.1) (type default)) (layer "Edge.Cuts"))
 (gr_arc (start 120.65 105.56875) (mid 117.84367 104.40633) (end 116.68125 101.6) (stroke (width 0.1) (type default)) (layer "Edge.Cuts"))
 (gr_arc (start 116.681251 87.312499) (mid 117.843671 84.50617) (end 120.65 83.34375) (stroke (width 0.1) (type default))
  (layer "Edge.Cuts"))
 (gr_line (start 130.175 83.34375) (end 120.65 83.34375) (stroke (width 0.1) (type default)) (layer "Edge.Cuts"))
 (segment (start 121.304 95.63) (end 121.304 96.766) (width 0.25) (layer "F.Cu") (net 1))
 (segment (start 121.304 96.766) (end 121.38 96.842) (width 0.25) (layer "F.Cu") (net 1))
 (via (at 121.38 96.842) (size 0.8) (drill 0.4) (layers "F.Cu" "B.Cu") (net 1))
 (segment (start 125.304 95.7425) (end 124.0905 95.7425) (width 0.25) (layer "F.Cu") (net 2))
 (segment (start 124.0905 95.7425) (end 122.378 94.03) (width 0.25) (layer "F.Cu") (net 2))
 (segment (start 122.378 94.03) (end 121.304 94.03) (width 0.25) (layer "F.Cu") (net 2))
 (segment (start 127.463 86.695) (end 126.46 87.698) (width 0.25) (layer "F.Cu") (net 4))
 (segment (start 126.46 87.698) (end 126.46 92.7615) (width 0.25) (layer "F.Cu") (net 4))
 (segment (start 129 86.695) (end 127.463 86.695) (width 0.25) (layer "F.Cu") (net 4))
 (segment (start 126.46 92.7615) (end 125.304 93.9175) (width 0.25) (layer "F.Cu") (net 4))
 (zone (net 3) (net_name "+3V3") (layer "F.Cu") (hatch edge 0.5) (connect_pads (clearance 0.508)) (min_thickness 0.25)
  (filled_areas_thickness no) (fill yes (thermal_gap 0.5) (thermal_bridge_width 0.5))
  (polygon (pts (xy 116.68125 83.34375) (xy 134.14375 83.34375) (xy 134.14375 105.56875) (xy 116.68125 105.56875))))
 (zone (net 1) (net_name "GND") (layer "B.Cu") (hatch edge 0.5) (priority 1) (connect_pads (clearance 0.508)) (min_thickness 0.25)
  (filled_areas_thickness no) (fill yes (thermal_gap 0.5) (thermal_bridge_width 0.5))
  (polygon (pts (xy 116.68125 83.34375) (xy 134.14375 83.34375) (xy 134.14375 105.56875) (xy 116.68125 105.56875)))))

